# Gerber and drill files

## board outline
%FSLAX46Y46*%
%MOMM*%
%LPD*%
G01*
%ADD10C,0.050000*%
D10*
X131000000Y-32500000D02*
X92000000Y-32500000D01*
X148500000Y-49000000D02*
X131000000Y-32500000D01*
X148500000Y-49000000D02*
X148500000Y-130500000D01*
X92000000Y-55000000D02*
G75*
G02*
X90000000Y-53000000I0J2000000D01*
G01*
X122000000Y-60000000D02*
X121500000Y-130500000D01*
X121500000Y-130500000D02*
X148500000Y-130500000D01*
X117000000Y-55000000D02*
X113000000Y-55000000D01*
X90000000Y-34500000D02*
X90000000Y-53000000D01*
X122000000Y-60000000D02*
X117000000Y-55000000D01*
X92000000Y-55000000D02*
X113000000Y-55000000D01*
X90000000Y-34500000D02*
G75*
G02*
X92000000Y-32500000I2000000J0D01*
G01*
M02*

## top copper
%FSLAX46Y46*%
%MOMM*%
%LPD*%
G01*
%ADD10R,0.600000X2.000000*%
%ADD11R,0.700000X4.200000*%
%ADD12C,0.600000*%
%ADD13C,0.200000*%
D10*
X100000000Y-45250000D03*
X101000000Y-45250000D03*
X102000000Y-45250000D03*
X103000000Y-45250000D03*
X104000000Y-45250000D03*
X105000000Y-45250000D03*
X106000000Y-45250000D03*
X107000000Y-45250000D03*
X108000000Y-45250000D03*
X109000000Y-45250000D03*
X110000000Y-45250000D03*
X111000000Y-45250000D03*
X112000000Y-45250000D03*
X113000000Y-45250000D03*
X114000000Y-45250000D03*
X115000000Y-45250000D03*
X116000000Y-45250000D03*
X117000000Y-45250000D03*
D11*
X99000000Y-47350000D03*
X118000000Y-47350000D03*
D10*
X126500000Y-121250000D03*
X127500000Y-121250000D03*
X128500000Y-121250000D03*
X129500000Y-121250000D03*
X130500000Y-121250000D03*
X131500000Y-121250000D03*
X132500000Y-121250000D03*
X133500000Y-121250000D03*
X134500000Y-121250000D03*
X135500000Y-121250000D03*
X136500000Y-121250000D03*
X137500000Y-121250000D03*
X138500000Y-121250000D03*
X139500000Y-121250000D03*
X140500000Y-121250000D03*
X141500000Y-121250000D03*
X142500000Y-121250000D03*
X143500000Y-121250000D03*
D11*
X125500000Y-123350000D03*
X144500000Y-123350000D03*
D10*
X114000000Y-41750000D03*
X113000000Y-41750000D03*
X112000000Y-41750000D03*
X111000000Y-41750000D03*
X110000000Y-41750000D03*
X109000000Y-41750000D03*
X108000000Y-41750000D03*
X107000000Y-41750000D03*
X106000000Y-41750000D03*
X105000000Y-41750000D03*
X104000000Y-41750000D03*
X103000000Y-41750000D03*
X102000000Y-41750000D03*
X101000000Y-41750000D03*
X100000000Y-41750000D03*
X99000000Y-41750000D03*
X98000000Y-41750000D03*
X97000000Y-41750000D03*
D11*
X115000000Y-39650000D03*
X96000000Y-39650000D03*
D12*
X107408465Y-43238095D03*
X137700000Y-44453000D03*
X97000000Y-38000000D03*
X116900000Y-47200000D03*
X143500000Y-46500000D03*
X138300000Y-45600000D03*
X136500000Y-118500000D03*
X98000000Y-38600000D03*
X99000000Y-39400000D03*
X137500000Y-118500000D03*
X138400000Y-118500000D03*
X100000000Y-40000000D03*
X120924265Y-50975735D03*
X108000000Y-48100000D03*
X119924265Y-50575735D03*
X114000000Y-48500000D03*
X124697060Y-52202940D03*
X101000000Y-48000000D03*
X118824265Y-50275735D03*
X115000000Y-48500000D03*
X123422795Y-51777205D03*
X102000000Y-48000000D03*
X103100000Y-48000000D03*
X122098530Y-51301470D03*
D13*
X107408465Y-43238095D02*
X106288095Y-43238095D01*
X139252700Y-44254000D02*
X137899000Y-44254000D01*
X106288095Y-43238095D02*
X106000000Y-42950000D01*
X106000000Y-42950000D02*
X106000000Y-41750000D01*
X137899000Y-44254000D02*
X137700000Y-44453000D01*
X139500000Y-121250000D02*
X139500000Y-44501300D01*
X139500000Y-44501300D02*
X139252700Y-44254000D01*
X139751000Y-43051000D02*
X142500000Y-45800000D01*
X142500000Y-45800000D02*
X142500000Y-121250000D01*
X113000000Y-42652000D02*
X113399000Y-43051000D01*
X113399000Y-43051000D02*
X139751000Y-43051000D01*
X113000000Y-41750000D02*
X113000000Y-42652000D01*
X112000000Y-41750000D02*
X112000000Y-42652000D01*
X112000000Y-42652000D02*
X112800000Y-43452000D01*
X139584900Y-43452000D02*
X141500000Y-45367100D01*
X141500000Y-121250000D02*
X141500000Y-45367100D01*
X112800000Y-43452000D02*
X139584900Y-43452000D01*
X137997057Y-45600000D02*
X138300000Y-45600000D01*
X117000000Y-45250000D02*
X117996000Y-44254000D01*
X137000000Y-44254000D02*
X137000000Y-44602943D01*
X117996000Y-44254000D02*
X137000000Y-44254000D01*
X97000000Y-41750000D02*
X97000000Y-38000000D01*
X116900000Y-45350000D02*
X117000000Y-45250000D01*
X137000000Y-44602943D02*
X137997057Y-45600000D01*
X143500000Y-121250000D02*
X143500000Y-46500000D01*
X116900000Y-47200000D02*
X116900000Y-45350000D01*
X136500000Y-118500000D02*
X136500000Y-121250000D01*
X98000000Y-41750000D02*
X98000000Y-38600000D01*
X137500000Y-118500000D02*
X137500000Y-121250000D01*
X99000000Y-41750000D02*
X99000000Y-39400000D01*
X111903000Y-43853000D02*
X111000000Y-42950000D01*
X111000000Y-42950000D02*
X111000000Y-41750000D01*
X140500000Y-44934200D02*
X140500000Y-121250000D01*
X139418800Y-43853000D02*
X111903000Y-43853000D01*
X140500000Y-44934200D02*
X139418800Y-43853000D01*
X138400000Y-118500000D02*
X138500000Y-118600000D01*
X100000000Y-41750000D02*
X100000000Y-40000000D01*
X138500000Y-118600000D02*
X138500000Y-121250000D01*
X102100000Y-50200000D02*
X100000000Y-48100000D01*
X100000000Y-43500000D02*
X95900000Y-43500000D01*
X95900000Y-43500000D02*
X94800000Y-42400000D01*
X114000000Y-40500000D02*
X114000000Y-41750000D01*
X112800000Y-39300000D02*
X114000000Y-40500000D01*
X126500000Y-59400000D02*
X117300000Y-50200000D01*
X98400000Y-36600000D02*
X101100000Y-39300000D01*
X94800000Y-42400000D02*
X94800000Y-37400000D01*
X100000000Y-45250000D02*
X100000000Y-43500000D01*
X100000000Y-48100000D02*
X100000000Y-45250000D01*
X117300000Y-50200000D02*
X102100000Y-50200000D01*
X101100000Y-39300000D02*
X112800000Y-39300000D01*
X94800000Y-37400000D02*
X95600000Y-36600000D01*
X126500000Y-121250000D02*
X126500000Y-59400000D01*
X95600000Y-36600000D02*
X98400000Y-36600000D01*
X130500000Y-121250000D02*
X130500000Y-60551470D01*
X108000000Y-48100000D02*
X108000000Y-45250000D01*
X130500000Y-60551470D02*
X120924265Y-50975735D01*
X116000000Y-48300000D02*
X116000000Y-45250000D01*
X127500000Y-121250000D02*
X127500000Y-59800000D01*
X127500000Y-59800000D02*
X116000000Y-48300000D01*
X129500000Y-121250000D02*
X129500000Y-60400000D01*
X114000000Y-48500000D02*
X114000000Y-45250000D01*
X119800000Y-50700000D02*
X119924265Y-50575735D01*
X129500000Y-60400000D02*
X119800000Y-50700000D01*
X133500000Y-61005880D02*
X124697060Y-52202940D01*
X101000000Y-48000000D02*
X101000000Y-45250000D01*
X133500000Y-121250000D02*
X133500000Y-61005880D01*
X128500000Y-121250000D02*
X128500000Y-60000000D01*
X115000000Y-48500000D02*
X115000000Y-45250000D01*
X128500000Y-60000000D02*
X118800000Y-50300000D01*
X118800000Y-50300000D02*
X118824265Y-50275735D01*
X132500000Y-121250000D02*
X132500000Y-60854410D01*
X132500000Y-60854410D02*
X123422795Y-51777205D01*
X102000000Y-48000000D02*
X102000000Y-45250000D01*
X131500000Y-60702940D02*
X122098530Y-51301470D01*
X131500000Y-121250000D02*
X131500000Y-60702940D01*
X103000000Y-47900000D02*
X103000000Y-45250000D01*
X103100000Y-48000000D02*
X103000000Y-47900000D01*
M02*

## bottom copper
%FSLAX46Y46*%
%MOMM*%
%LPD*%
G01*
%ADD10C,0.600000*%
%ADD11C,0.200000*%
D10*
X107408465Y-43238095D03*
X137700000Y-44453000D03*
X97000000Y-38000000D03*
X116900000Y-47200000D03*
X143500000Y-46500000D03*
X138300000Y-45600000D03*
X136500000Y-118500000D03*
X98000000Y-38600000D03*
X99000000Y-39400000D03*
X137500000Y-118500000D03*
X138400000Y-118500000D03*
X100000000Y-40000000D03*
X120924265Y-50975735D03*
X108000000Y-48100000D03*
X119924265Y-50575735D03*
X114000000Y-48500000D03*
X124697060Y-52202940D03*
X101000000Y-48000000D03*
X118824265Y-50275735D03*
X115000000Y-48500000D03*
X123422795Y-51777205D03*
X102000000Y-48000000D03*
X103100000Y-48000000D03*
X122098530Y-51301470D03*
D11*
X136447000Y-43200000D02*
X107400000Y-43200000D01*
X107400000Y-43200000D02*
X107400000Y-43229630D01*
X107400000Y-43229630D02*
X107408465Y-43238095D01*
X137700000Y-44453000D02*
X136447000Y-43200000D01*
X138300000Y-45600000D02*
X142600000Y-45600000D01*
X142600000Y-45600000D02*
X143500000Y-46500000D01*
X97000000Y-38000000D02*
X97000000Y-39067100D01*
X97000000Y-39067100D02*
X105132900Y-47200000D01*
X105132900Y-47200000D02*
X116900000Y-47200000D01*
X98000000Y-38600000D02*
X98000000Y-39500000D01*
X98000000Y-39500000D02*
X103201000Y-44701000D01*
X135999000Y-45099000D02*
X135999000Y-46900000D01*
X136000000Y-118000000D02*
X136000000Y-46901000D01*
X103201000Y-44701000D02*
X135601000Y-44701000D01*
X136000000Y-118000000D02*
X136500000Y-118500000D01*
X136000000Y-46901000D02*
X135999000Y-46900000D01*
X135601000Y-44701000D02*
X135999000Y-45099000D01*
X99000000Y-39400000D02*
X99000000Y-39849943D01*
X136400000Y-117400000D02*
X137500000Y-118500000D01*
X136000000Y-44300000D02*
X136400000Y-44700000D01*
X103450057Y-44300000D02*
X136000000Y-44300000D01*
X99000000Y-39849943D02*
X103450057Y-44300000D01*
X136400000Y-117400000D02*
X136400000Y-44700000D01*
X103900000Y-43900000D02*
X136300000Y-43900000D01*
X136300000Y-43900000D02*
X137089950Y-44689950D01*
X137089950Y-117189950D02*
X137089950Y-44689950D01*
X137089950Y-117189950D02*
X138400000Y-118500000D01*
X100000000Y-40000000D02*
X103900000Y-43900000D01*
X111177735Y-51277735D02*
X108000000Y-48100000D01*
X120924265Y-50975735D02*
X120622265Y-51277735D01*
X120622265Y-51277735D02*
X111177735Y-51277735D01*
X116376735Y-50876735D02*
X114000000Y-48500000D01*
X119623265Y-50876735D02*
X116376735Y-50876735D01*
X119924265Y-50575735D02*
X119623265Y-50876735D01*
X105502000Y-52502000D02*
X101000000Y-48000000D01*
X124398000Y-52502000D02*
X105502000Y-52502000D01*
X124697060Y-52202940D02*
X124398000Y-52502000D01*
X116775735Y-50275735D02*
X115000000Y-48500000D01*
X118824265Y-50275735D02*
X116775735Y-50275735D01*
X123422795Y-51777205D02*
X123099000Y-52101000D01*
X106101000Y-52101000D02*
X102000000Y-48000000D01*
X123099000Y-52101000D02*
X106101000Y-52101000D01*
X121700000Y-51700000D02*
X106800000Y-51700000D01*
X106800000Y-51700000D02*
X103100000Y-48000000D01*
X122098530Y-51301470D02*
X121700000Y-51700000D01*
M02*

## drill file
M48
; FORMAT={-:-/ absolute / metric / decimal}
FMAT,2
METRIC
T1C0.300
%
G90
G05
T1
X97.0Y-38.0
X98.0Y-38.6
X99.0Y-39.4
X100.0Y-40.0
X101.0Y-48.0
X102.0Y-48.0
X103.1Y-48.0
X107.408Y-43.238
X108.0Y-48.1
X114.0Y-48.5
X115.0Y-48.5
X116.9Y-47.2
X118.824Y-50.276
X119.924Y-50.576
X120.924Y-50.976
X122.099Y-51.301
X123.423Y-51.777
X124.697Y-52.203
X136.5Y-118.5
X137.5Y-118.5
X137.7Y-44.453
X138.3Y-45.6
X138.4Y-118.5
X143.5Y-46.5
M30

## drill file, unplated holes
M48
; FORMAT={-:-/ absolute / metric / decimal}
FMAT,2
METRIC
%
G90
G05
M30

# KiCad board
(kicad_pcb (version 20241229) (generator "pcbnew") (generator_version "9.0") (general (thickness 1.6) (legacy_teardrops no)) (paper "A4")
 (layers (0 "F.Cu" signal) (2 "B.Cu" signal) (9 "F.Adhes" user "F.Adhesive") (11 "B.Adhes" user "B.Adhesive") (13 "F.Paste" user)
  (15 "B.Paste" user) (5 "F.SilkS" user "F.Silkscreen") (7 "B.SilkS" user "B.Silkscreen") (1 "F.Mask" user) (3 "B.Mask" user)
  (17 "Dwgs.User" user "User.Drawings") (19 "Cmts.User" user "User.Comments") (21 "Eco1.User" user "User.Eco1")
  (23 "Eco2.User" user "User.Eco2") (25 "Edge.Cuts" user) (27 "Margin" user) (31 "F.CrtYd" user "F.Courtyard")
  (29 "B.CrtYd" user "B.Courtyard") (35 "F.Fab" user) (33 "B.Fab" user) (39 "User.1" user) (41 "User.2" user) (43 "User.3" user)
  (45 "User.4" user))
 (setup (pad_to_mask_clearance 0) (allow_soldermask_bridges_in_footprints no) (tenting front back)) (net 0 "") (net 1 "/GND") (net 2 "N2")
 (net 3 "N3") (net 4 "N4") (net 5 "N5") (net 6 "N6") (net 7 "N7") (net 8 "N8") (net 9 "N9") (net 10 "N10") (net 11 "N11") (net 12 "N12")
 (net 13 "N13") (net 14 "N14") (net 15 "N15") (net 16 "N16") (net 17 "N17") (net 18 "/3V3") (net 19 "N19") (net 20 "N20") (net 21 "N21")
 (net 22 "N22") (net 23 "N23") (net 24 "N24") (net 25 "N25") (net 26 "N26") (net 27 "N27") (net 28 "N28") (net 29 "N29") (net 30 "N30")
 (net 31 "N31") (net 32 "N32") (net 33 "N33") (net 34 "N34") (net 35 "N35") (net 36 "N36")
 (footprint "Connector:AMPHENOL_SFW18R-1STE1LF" (layer "F.Cu") (at 108.5 48.5)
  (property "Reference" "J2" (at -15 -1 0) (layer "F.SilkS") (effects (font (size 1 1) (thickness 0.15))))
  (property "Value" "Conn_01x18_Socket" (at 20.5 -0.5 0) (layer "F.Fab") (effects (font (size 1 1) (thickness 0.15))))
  (pad "1" smd rect (at -8.5 -3.25) (size 0.6 2) (layers "F.Cu" "F.Mask" "F.Paste") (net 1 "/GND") (solder_mask_margin 0.102))
  (pad "2" smd rect (at -7.5 -3.25) (size 0.6 2) (layers "F.Cu" "F.Mask" "F.Paste") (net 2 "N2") (solder_mask_margin 0.102))
  (pad "3" smd rect (at -6.5 -3.25) (size 0.6 2) (layers "F.Cu" "F.Mask" "F.Paste") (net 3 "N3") (solder_mask_margin 0.102))
  (pad "4" smd rect (at -5.5 -3.25) (size 0.6 2) (layers "F.Cu" "F.Mask" "F.Paste") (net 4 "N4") (solder_mask_margin 0.102))
  (pad "5" smd rect (at -4.5 -3.25) (size 0.6 2) (layers "F.Cu" "F.Mask" "F.Paste") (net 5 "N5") (solder_mask_margin 0.102))
  (pad "6" smd rect (at -3.5 -3.25) (size 0.6 2) (layers "F.Cu" "F.Mask" "F.Paste") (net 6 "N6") (solder_mask_margin 0.102))
  (pad "7" smd rect (at -2.5 -3.25) (size 0.6 2) (layers "F.Cu" "F.Mask" "F.Paste") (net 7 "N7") (solder_mask_margin 0.102))
  (pad "8" smd rect (at -1.5 -3.25) (size 0.6 2) (layers "F.Cu" "F.Mask" "F.Paste") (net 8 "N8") (solder_mask_margin 0.102))
  (pad "9" smd rect (at -0.5 -3.25) (size 0.6 2) (layers "F.Cu" "F.Mask" "F.Paste") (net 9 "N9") (solder_mask_margin 0.102))
  (pad "10" smd rect (at 0.5 -3.25) (size 0.6 2) (layers "F.Cu" "F.Mask" "F.Paste") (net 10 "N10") (solder_mask_margin 0.102))
  (pad "11" smd rect (at 1.5 -3.25) (size 0.6 2) (layers "F.Cu" "F.Mask" "F.Paste") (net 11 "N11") (solder_mask_margin 0.102))
  (pad "12" smd rect (at 2.5 -3.25) (size 0.6 2) (layers "F.Cu" "F.Mask" "F.Paste") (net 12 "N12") (solder_mask_margin 0.102))
  (pad "13" smd rect (at 3.5 -3.25) (size 0.6 2) (layers "F.Cu" "F.Mask" "F.Paste") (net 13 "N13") (solder_mask_margin 0.102))
  (pad "14" smd rect (at 4.5 -3.25) (size 0.6 2) (layers "F.Cu" "F.Mask" "F.Paste") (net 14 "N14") (solder_mask_margin 0.102))
  (pad "15" smd rect (at 5.5 -3.25) (size 0.6 2) (layers "F.Cu" "F.Mask" "F.Paste") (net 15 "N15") (solder_mask_margin 0.102))
  (pad "16" smd rect (at 6.5 -3.25) (size 0.6 2) (layers "F.Cu" "F.Mask" "F.Paste") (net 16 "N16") (solder_mask_margin 0.102))
  (pad "17" smd rect (at 7.5 -3.25) (size 0.6 2) (layers "F.Cu" "F.Mask" "F.Paste") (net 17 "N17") (solder_mask_margin 0.102))
  (pad "18" smd rect (at 8.5 -3.25) (size 0.6 2) (layers "F.Cu" "F.Mask" "F.Paste") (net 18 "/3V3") (solder_mask_margin 0.102))
  (pad "S1" smd rect (at -9.5 -1.15) (size 0.7 4.2) (layers "F.Cu" "F.Mask" "F.Paste") (solder_mask_margin 0.102))
  (pad "S2" smd rect (at 9.5 -1.15) (size 0.7 4.2) (layers "F.Cu" "F.Mask" "F.Paste") (solder_mask_margin 0.102)))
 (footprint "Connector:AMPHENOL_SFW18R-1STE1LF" (layer "F.Cu") (at 135 124.5)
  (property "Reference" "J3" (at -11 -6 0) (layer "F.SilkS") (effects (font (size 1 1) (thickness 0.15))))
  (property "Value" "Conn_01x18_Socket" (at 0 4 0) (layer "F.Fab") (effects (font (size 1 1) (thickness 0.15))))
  (pad "1" smd rect (at -8.5 -3.25) (size 0.6 2) (layers "F.Cu" "F.Mask" "F.Paste") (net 1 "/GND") (solder_mask_margin 0.102))
  (pad "2" smd rect (at -7.5 -3.25) (size 0.6 2) (layers "F.Cu" "F.Mask" "F.Paste") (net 17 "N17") (solder_mask_margin 0.102))
  (pad "3" smd rect (at -6.5 -3.25) (size 0.6 2) (layers "F.Cu" "F.Mask" "F.Paste") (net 16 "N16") (solder_mask_margin 0.102))
  (pad "4" smd rect (at -5.5 -3.25) (size 0.6 2) (layers "F.Cu" "F.Mask" "F.Paste") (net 15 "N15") (solder_mask_margin 0.102))
  (pad "5" smd rect (at -4.5 -3.25) (size 0.6 2) (layers "F.Cu" "F.Mask" "F.Paste") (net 9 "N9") (solder_mask_margin 0.102))
  (pad "6" smd rect (at -3.5 -3.25) (size 0.6 2) (layers "F.Cu" "F.Mask" "F.Paste") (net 4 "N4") (solder_mask_margin 0.102))
  (pad "7" smd rect (at -2.5 -3.25) (size 0.6 2) (layers "F.Cu" "F.Mask" "F.Paste") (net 3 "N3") (solder_mask_margin 0.102))
  (pad "8" smd rect (at -1.5 -3.25) (size 0.6 2) (layers "F.Cu" "F.Mask" "F.Paste") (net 2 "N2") (solder_mask_margin 0.102))
  (pad "9" smd rect (at -0.5 -3.25) (size 0.6 2) (layers "F.Cu" "F.Mask" "F.Paste") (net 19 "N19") (solder_mask_margin 0.102))
  (pad "10" smd rect (at 0.5 -3.25) (size 0.6 2) (layers "F.Cu" "F.Mask" "F.Paste") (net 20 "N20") (solder_mask_margin 0.102))
  (pad "11" smd rect (at 1.5 -3.25) (size 0.6 2) (layers "F.Cu" "F.Mask" "F.Paste") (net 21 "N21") (solder_mask_margin 0.102))
  (pad "12" smd rect (at 2.5 -3.25) (size 0.6 2) (layers "F.Cu" "F.Mask" "F.Paste") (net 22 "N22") (solder_mask_margin 0.102))
  (pad "13" smd rect (at 3.5 -3.25) (size 0.6 2) (layers "F.Cu" "F.Mask" "F.Paste") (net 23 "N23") (solder_mask_margin 0.102))
  (pad "14" smd rect (at 4.5 -3.25) (size 0.6 2) (layers "F.Cu" "F.Mask" "F.Paste") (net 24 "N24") (solder_mask_margin 0.102))
  (pad "15" smd rect (at 5.5 -3.25) (size 0.6 2) (layers "F.Cu" "F.Mask" "F.Paste") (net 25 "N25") (solder_mask_margin 0.102))
  (pad "16" smd rect (at 6.5 -3.25) (size 0.6 2) (layers "F.Cu" "F.Mask" "F.Paste") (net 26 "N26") (solder_mask_margin 0.102))
  (pad "17" smd rect (at 7.5 -3.25) (size 0.6 2) (layers "F.Cu" "F.Mask" "F.Paste") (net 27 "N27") (solder_mask_margin 0.102))
  (pad "18" smd rect (at 8.5 -3.25) (size 0.6 2) (layers "F.Cu" "F.Mask" "F.Paste") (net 18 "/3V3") (solder_mask_margin 0.102))
  (pad "S1" smd rect (at -9.5 -1.15) (size 0.7 4.2) (layers "F.Cu" "F.Mask" "F.Paste") (solder_mask_margin 0.102))
  (pad "S2" smd rect (at 9.5 -1.15) (size 0.7 4.2) (layers "F.Cu" "F.Mask" "F.Paste") (solder_mask_margin 0.102)))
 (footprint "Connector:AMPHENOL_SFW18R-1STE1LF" (layer "F.Cu") (at 105.5 38.5 180)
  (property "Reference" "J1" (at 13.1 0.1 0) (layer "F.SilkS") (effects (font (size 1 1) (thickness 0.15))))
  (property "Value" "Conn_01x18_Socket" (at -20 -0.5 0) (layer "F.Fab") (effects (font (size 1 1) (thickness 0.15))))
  (pad "1" smd rect (at -8.5 -3.25 180) (size 0.6 2) (layers "F.Cu" "F.Mask" "F.Paste") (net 1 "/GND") (solder_mask_margin 0.102))
  (pad "2" smd rect (at -7.5 -3.25 180) (size 0.6 2) (layers "F.Cu" "F.Mask" "F.Paste") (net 27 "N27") (solder_mask_margin 0.102))
  (pad "3" smd rect (at -6.5 -3.25 180) (size 0.6 2) (layers "F.Cu" "F.Mask" "F.Paste") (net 26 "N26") (solder_mask_margin 0.102))
  (pad "4" smd rect (at -5.5 -3.25 180) (size 0.6 2) (layers "F.Cu" "F.Mask" "F.Paste") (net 25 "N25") (solder_mask_margin 0.102))
  (pad "5" smd rect (at -4.5 -3.25 180) (size 0.6 2) (layers "F.Cu" "F.Mask" "F.Paste") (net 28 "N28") (solder_mask_margin 0.102))
  (pad "6" smd rect (at -3.5 -3.25 180) (size 0.6 2) (layers "F.Cu" "F.Mask" "F.Paste") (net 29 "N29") (solder_mask_margin 0.102))
  (pad "7" smd rect (at -2.5 -3.25 180) (size 0.6 2) (layers "F.Cu" "F.Mask" "F.Paste") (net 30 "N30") (solder_mask_margin 0.102))
  (pad "8" smd rect (at -1.5 -3.25 180) (size 0.6 2) (layers "F.Cu" "F.Mask" "F.Paste") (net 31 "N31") (solder_mask_margin 0.102))
  (pad "9" smd rect (at -0.5 -3.25 180) (size 0.6 2) (layers "F.Cu" "F.Mask" "F.Paste") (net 24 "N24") (solder_mask_margin 0.102))
  (pad "10" smd rect (at 0.5 -3.25 180) (size 0.6 2) (layers "F.Cu" "F.Mask" "F.Paste") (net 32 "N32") (solder_mask_margin 0.102))
  (pad "11" smd rect (at 1.5 -3.25 180) (size 0.6 2) (layers "F.Cu" "F.Mask" "F.Paste") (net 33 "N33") (solder_mask_margin 0.102))
  (pad "12" smd rect (at 2.5 -3.25 180) (size 0.6 2) (layers "F.Cu" "F.Mask" "F.Paste") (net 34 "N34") (solder_mask_margin 0.102))
  (pad "13" smd rect (at 3.5 -3.25 180) (size 0.6 2) (layers "F.Cu" "F.Mask" "F.Paste") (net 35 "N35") (solder_mask_margin 0.102))
  (pad "14" smd rect (at 4.5 -3.25 180) (size 0.6 2) (layers "F.Cu" "F.Mask" "F.Paste") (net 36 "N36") (solder_mask_margin 0.102))
  (pad "15" smd rect (at 5.5 -3.25 180) (size 0.6 2) (layers "F.Cu" "F.Mask" "F.Paste") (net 23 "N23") (solder_mask_margin 0.102))
  (pad "16" smd rect (at 6.5 -3.25 180) (size 0.6 2) (layers "F.Cu" "F.Mask" "F.Paste") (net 22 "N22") (solder_mask_margin 0.102))
  (pad "17" smd rect (at 7.5 -3.25 180) (size 0.6 2) (layers "F.Cu" "F.Mask" "F.Paste") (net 21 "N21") (solder_mask_margin 0.102))
  (pad "18" smd rect (at 8.5 -3.25 180) (size 0.6 2) (layers "F.Cu" "F.Mask" "F.Paste") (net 18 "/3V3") (solder_mask_margin 0.102))
  (pad "S1" smd rect (at -9.5 -1.15 180) (size 0.7 4.2) (layers "F.Cu" "F.Mask" "F.Paste") (solder_mask_margin 0.102))
  (pad "S2" smd rect (at 9.5 -1.15 180) (size 0.7 4.2) (layers "F.Cu" "F.Mask" "F.Paste") (solder_mask_margin 0.102)))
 (gr_line (start 131 32.5) (end 92 32.5) (stroke (width 0.05) (type default)) (layer "Edge.Cuts"))
 (gr_line (start 148.5 49) (end 131 32.5) (stroke (width 0.05) (type default)) (layer "Edge.Cuts"))
 (gr_line (start 148.5 49) (end 148.5 130.5) (stroke (width 0.05) (type default)) (layer "Edge.Cuts"))
 (gr_arc (start 92 55) (mid 90.585786 54.414214) (end 90 53) (stroke (width 0.05) (type default)) (layer "Edge.Cuts"))
 (gr_line (start 122 60) (end 121.5 130.5) (stroke (width 0.05) (type default)) (layer "Edge.Cuts"))
 (gr_line (start 121.5 130.5) (end 148.5 130.5) (stroke (width 0.05) (type default)) (layer "Edge.Cuts"))
 (gr_line (start 117 55) (end 113 55) (stroke (width 0.05) (type default)) (layer "Edge.Cuts"))
 (gr_line (start 90 34.5) (end 90 53) (stroke (width 0.05) (type default)) (layer "Edge.Cuts"))
 (gr_line (start 122 60) (end 117 55) (stroke (width 0.05) (type default)) (layer "Edge.Cuts"))
 (gr_line (start 92 55) (end 113 55) (stroke (width 0.05) (type default)) (layer "Edge.Cuts"))
 (gr_arc (start 90 34.5) (mid 90.585786 33.085786) (end 92 32.5) (stroke (width 0.05) (type default)) (layer "Edge.Cuts"))
 (segment (start 107.408465 43.238095) (end 106.288095 43.238095) (width 0.2) (layer "F.Cu") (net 24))
 (segment (start 139.2527 44.254) (end 137.899 44.254) (width 0.2) (layer "F.Cu") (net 24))
 (segment (start 106.288095 43.238095) (end 106 42.95) (width 0.2) (layer "F.Cu") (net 24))
 (segment (start 106 42.95) (end 106 41.75) (width 0.2) (layer "F.Cu") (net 24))
 (segment (start 137.899 44.254) (end 137.7 44.453) (width 0.2) (layer "F.Cu") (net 24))
 (segment (start 139.5 121.25) (end 139.5 44.5013) (width 0.2) (layer "F.Cu") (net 24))
 (segment (start 139.5 44.5013) (end 139.2527 44.254) (width 0.2) (layer "F.Cu") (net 24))
 (via (at 107.408465 43.238095) (size 0.6) (drill 0.3) (layers "F.Cu" "B.Cu") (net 24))
 (via (at 137.7 44.453) (size 0.6) (drill 0.3) (layers "F.Cu" "B.Cu") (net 24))
 (segment (start 136.447 43.2) (end 107.4 43.2) (width 0.2) (layer "B.Cu") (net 24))
 (segment (start 107.4 43.2) (end 107.4 43.22963) (width 0.2) (layer "B.Cu") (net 24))
 (segment (start 107.4 43.22963) (end 107.408465 43.238095) (width 0.2) (layer "B.Cu") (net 24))
 (segment (start 137.7 44.453) (end 136.447 43.2) (width 0.2) (layer "B.Cu") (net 24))
 (segment (start 139.751 43.051) (end 142.5 45.8) (width 0.2) (layer "F.Cu") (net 27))
 (segment (start 142.5 45.8) (end 142.5 121.25) (width 0.2) (layer "F.Cu") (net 27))
 (segment (start 113 42.652) (end 113.399 43.051) (width 0.2) (layer "F.Cu") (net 27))
 (segment (start 113.399 43.051) (end 139.751 43.051) (width 0.2) (layer "F.Cu") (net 27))
 (segment (start 113 41.75) (end 113 42.652) (width 0.2) (layer "F.Cu") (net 27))
 (segment (start 112 41.75) (end 112 42.652) (width 0.2) (layer "F.Cu") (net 26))
 (segment (start 112 42.652) (end 112.8 43.452) (width 0.2) (layer "F.Cu") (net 26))
 (segment (start 139.5849 43.452) (end 141.5 45.3671) (width 0.2) (layer "F.Cu") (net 26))
 (segment (start 141.5 121.25) (end 141.5 45.3671) (width 0.2) (layer "F.Cu") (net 26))
 (segment (start 112.8 43.452) (end 139.5849 43.452) (width 0.2) (layer "F.Cu") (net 26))
 (segment (start 137.997057 45.6) (end 138.3 45.6) (width 0.2) (layer "F.Cu") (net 18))
 (segment (start 117 45.25) (end 117.996 44.254) (width 0.2) (layer "F.Cu") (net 18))
 (segment (start 137 44.254) (end 137 44.602943) (width 0.2) (layer "F.Cu") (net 18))
 (segment (start 117.996 44.254) (end 137 44.254) (width 0.2) (layer "F.Cu") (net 18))
 (segment (start 97 41.75) (end 97 38) (width 0.2) (layer "F.Cu") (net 18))
 (segment (start 116.9 45.35) (end 117 45.25) (width 0.2) (layer "F.Cu") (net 18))
 (segment (start 137 44.602943) (end 137.997057 45.6) (width 0.2) (layer "F.Cu") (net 18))
 (segment (start 143.5 121.25) (end 143.5 46.5) (width 0.2) (layer "F.Cu") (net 18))
 (segment (start 116.9 47.2) (end 116.9 45.35) (width 0.2) (layer "F.Cu") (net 18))
 (via (at 97 38) (size 0.6) (drill 0.3) (layers "F.Cu" "B.Cu") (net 18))
 (via (at 116.9 47.2) (size 0.6) (drill 0.3) (layers "F.Cu" "B.Cu") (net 18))
 (via (at 143.5 46.5) (size 0.6) (drill 0.3) (layers "F.Cu" "B.Cu") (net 18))
 (via (at 138.3 45.6) (size 0.6) (drill 0.3) (layers "F.Cu" "B.Cu") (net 18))
 (segment (start 138.3 45.6) (end 142.6 45.6) (width 0.2) (layer "B.Cu") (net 18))
 (segment (start 142.6 45.6) (end 143.5 46.5) (width 0.2) (layer "B.Cu") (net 18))
 (segment (start 97 38) (end 97 39.0671) (width 0.2) (layer "B.Cu") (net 18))
 (segment (start 97 39.0671) (end 105.1329 47.2) (width 0.2) (layer "B.Cu") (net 18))
 (segment (start 105.1329 47.2) (end 116.9 47.2) (width 0.2) (layer "B.Cu") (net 18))
 (segment (start 136.5 118.5) (end 136.5 121.25) (width 0.2) (layer "F.Cu") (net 21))
 (segment (start 98 41.75) (end 98 38.6) (width 0.2) (layer "F.Cu") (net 21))
 (via (at 136.5 118.5) (size 0.6) (drill 0.3) (layers "F.Cu" "B.Cu") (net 21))
 (via (at 98 38.6) (size 0.6) (drill 0.3) (layers "F.Cu" "B.Cu") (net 21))
 (segment (start 98 38.6) (end 98 39.5) (width 0.2) (layer "B.Cu") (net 21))
 (segment (start 98 39.5) (end 103.201 44.701) (width 0.2) (layer "B.Cu") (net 21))
 (segment (start 135.999 45.099) (end 135.999 46.9) (width 0.2) (layer "B.Cu") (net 21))
 (segment (start 136 118) (end 136 46.901) (width 0.2) (layer "B.Cu") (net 21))
 (segment (start 103.201 44.701) (end 135.601 44.701) (width 0.2) (layer "B.Cu") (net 21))
 (segment (start 136 118) (end 136.5 118.5) (width 0.2) (layer "B.Cu") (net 21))
 (segment (start 136 46.901) (end 135.999 46.9) (width 0.2) (layer "B.Cu") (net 21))
 (segment (start 135.601 44.701) (end 135.999 45.099) (width 0.2) (layer "B.Cu") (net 21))
 (segment (start 137.5 118.5) (end 137.5 121.25) (width 0.2) (layer "F.Cu") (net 22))
 (segment (start 99 41.75) (end 99 39.4) (width 0.2) (layer "F.Cu") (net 22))
 (via (at 99 39.4) (size 0.6) (drill 0.3) (layers "F.Cu" "B.Cu") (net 22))
 (via (at 137.5 118.5) (size 0.6) (drill 0.3) (layers "F.Cu" "B.Cu") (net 22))
 (segment (start 99 39.4) (end 99 39.849943) (width 0.2) (layer "B.Cu") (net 22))
 (segment (start 136.4 117.4) (end 137.5 118.5) (width 0.2) (layer "B.Cu") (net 22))
 (segment (start 136 44.3) (end 136.4 44.7) (width 0.2) (layer "B.Cu") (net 22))
 (segment (start 103.450057 44.3) (end 136 44.3) (width 0.2) (layer "B.Cu") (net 22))
 (segment (start 99 39.849943) (end 103.450057 44.3) (width 0.2) (layer "B.Cu") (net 22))
 (segment (start 136.4 117.4) (end 136.4 44.7) (width 0.2) (layer "B.Cu") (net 22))
 (segment (start 111.903 43.853) (end 111 42.95) (width 0.2) (layer "F.Cu") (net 25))
 (segment (start 111 42.95) (end 111 41.75) (width 0.2) (layer "F.Cu") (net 25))
 (segment (start 140.5 44.9342) (end 140.5 121.25) (width 0.2) (layer "F.Cu") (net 25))
 (segment (start 139.4188 43.853) (end 111.903 43.853) (width 0.2) (layer "F.Cu") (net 25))
 (segment (start 140.5 44.9342) (end 139.4188 43.853) (width 0.2) (layer "F.Cu") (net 25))
 (segment (start 138.4 118.5) (end 138.5 118.6) (width 0.2) (layer "F.Cu") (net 23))
 (segment (start 100 41.75) (end 100 40) (width 0.2) (layer "F.Cu") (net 23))
 (segment (start 138.5 118.6) (end 138.5 121.25) (width 0.2) (layer "F.Cu") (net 23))
 (via (at 138.4 118.5) (size 0.6) (drill 0.3) (layers "F.Cu" "B.Cu") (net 23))
 (via (at 100 40) (size 0.6) (drill 0.3) (layers "F.Cu" "B.Cu") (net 23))
 (segment (start 103.9 43.9) (end 136.3 43.9) (width 0.2) (layer "B.Cu") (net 23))
 (segment (start 136.3 43.9) (end 137.08995 44.68995) (width 0.2) (layer "B.Cu") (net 23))
 (segment (start 137.08995 117.18995) (end 137.08995 44.68995) (width 0.2) (layer "B.Cu") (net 23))
 (segment (start 137.08995 117.18995) (end 138.4 118.5) (width 0.2) (layer "B.Cu") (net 23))
 (segment (start 100 40) (end 103.9 43.9) (width 0.2) (layer "B.Cu") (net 23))
 (segment (start 102.1 50.2) (end 100 48.1) (width 0.2) (layer "F.Cu") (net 1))
 (segment (start 100 43.5) (end 95.9 43.5) (width 0.2) (layer "F.Cu") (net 1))
 (segment (start 95.9 43.5) (end 94.8 42.4) (width 0.2) (layer "F.Cu") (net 1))
 (segment (start 114 40.5) (end 114 41.75) (width 0.2) (layer "F.Cu") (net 1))
 (segment (start 112.8 39.3) (end 114 40.5) (width 0.2) (layer "F.Cu") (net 1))
 (segment (start 126.5 59.4) (end 117.3 50.2) (width 0.2) (layer "F.Cu") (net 1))
 (segment (start 98.4 36.6) (end 101.1 39.3) (width 0.2) (layer "F.Cu") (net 1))
 (segment (start 94.8 42.4) (end 94.8 37.4) (width 0.2) (layer "F.Cu") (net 1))
 (segment (start 100 45.25) (end 100 43.5) (width 0.2) (layer "F.Cu") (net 1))
 (segment (start 100 48.1) (end 100 45.25) (width 0.2) (layer "F.Cu") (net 1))
 (segment (start 117.3 50.2) (end 102.1 50.2) (width 0.2) (layer "F.Cu") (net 1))
 (segment (start 101.1 39.3) (end 112.8 39.3) (width 0.2) (layer "F.Cu") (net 1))
 (segment (start 94.8 37.4) (end 95.6 36.6) (width 0.2) (layer "F.Cu") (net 1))
 (segment (start 126.5 121.25) (end 126.5 59.4) (width 0.2) (layer "F.Cu") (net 1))
 (segment (start 95.6 36.6) (end 98.4 36.6) (width 0.2) (layer "F.Cu") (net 1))
 (segment (start 130.5 121.25) (end 130.5 60.55147) (width 0.2) (layer "F.Cu") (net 9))
 (segment (start 108 48.1) (end 108 45.25) (width 0.2) (layer "F.Cu") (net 9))
 (segment (start 130.5 60.55147) (end 120.924265 50.975735) (width 0.2) (layer "F.Cu") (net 9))
 (via (at 120.924265 50.975735) (size 0.6) (drill 0.3) (layers "F.Cu" "B.Cu") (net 9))
 (via (at 108 48.1) (size 0.6) (drill 0.3) (layers "F.Cu" "B.Cu") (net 9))
 (segment (start 111.177735 51.277735) (end 108 48.1) (width 0.2) (layer "B.Cu") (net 9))
 (segment (start 120.924265 50.975735) (end 120.622265 51.277735) (width 0.2) (layer "B.Cu") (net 9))
 (segment (start 120.622265 51.277735) (end 111.177735 51.277735) (width 0.2) (layer "B.Cu") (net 9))
 (segment (start 116 48.3) (end 116 45.25) (width 0.2) (layer "F.Cu") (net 17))
 (segment (start 127.5 121.25) (end 127.5 59.8) (width 0.2) (layer "F.Cu") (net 17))
 (segment (start 127.5 59.8) (end 116 48.3) (width 0.2) (layer "F.Cu") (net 17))
 (segment (start 129.5 121.25) (end 129.5 60.4) (width 0.2) (layer "F.Cu") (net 15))
 (segment (start 114 48.5) (end 114 45.25) (width 0.2) (layer "F.Cu") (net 15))
 (segment (start 119.8 50.7) (end 119.924265 50.575735) (width 0.2) (layer "F.Cu") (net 15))
 (segment (start 129.5 60.4) (end 119.8 50.7) (width 0.2) (layer "F.Cu") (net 15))
 (via (at 119.924265 50.575735) (size 0.6) (drill 0.3) (layers "F.Cu" "B.Cu") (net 15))
 (via (at 114 48.5) (size 0.6) (drill 0.3) (layers "F.Cu" "B.Cu") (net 15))
 (segment (start 116.376735 50.876735) (end 114 48.5) (width 0.2) (layer "B.Cu") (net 15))
 (segment (start 119.623265 50.876735) (end 116.376735 50.876735) (width 0.2) (layer "B.Cu") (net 15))
 (segment (start 119.924265 50.575735) (end 119.623265 50.876735) (width 0.2) (layer "B.Cu") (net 15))
 (segment (start 133.5 61.00588) (end 124.69706 52.20294) (width 0.2) (layer "F.Cu") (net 2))
 (segment (start 101 48) (end 101 45.25) (width 0.2) (layer "F.Cu") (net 2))
 (segment (start 133.5 121.25) (end 133.5 61.00588) (width 0.2) (layer "F.Cu") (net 2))
 (via (at 124.69706 52.20294) (size 0.6) (drill 0.3) (layers "F.Cu" "B.Cu") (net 2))
 (via (at 101 48) (size 0.6) (drill 0.3) (layers "F.Cu" "B.Cu") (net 2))
 (segment (start 105.502 52.502) (end 101 48) (width 0.2) (layer "B.Cu") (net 2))
 (segment (start 124.398 52.502) (end 105.502 52.502) (width 0.2) (layer "B.Cu") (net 2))
 (segment (start 124.69706 52.20294) (end 124.398 52.502) (width 0.2) (layer "B.Cu") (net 2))
 (segment (start 128.5 121.25) (end 128.5 60) (width 0.2) (layer "F.Cu") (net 16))
 (segment (start 115 48.5) (end 115 45.25) (width 0.2) (layer "F.Cu") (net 16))
 (segment (start 128.5 60) (end 118.8 50.3) (width 0.2) (layer "F.Cu") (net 16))
 (segment (start 118.8 50.3) (end 118.824265 50.275735) (width 0.2) (layer "F.Cu") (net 16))
 (via (at 118.824265 50.275735) (size 0.6) (drill 0.3) (layers "F.Cu" "B.Cu") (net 16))
 (via (at 115 48.5) (size 0.6) (drill 0.3) (layers "F.Cu" "B.Cu") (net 16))
 (segment (start 116.775735 50.275735) (end 115 48.5) (width 0.2) (layer "B.Cu") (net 16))
 (segment (start 118.824265 50.275735) (end 116.775735 50.275735) (width 0.2) (layer "B.Cu") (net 16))
 (segment (start 132.5 121.25) (end 132.5 60.85441) (width 0.2) (layer "F.Cu") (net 3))
 (segment (start 132.5 60.85441) (end 123.422795 51.777205) (width 0.2) (layer "F.Cu") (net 3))
 (segment (start 102 48) (end 102 45.25) (width 0.2) (layer "F.Cu") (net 3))
 (via (at 123.422795 51.777205) (size 0.6) (drill 0.3) (layers "F.Cu" "B.Cu") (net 3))
 (via (at 102 48) (size 0.6) (drill 0.3) (layers "F.Cu" "B.Cu") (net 3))
 (segment (start 123.422795 51.777205) (end 123.099 52.101) (width 0.2) (layer "B.Cu") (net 3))
 (segment (start 106.101 52.101) (end 102 48) (width 0.2) (layer "B.Cu") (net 3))
 (segment (start 123.099 52.101) (end 106.101 52.101) (width 0.2) (layer "B.Cu") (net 3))
 (segment (start 131.5 60.70294) (end 122.09853 51.30147) (width 0.2) (layer "F.Cu") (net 4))
 (segment (start 131.5 121.25) (end 131.5 60.70294) (width 0.2) (layer "F.Cu") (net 4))
 (segment (start 103 47.9) (end 103 45.25) (width 0.2) (layer "F.Cu") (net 4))
 (segment (start 103.1 48) (end 103 47.9) (width 0.2) (layer "F.Cu") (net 4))
 (via (at 103.1 48) (size 0.6) (drill 0.3) (layers "F.Cu" "B.Cu") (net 4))
 (via (at 122.09853 51.30147) (size 0.6) (drill 0.3) (layers "F.Cu" "B.Cu") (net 4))
 (segment (start 121.7 51.7) (end 106.8 51.7) (width 0.2) (layer "B.Cu") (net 4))
 (segment (start 106.8 51.7) (end 103.1 48) (width 0.2) (layer "B.Cu") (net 4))
 (segment (start 122.09853 51.30147) (end 121.7 51.7) (width 0.2) (layer "B.Cu") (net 4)))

